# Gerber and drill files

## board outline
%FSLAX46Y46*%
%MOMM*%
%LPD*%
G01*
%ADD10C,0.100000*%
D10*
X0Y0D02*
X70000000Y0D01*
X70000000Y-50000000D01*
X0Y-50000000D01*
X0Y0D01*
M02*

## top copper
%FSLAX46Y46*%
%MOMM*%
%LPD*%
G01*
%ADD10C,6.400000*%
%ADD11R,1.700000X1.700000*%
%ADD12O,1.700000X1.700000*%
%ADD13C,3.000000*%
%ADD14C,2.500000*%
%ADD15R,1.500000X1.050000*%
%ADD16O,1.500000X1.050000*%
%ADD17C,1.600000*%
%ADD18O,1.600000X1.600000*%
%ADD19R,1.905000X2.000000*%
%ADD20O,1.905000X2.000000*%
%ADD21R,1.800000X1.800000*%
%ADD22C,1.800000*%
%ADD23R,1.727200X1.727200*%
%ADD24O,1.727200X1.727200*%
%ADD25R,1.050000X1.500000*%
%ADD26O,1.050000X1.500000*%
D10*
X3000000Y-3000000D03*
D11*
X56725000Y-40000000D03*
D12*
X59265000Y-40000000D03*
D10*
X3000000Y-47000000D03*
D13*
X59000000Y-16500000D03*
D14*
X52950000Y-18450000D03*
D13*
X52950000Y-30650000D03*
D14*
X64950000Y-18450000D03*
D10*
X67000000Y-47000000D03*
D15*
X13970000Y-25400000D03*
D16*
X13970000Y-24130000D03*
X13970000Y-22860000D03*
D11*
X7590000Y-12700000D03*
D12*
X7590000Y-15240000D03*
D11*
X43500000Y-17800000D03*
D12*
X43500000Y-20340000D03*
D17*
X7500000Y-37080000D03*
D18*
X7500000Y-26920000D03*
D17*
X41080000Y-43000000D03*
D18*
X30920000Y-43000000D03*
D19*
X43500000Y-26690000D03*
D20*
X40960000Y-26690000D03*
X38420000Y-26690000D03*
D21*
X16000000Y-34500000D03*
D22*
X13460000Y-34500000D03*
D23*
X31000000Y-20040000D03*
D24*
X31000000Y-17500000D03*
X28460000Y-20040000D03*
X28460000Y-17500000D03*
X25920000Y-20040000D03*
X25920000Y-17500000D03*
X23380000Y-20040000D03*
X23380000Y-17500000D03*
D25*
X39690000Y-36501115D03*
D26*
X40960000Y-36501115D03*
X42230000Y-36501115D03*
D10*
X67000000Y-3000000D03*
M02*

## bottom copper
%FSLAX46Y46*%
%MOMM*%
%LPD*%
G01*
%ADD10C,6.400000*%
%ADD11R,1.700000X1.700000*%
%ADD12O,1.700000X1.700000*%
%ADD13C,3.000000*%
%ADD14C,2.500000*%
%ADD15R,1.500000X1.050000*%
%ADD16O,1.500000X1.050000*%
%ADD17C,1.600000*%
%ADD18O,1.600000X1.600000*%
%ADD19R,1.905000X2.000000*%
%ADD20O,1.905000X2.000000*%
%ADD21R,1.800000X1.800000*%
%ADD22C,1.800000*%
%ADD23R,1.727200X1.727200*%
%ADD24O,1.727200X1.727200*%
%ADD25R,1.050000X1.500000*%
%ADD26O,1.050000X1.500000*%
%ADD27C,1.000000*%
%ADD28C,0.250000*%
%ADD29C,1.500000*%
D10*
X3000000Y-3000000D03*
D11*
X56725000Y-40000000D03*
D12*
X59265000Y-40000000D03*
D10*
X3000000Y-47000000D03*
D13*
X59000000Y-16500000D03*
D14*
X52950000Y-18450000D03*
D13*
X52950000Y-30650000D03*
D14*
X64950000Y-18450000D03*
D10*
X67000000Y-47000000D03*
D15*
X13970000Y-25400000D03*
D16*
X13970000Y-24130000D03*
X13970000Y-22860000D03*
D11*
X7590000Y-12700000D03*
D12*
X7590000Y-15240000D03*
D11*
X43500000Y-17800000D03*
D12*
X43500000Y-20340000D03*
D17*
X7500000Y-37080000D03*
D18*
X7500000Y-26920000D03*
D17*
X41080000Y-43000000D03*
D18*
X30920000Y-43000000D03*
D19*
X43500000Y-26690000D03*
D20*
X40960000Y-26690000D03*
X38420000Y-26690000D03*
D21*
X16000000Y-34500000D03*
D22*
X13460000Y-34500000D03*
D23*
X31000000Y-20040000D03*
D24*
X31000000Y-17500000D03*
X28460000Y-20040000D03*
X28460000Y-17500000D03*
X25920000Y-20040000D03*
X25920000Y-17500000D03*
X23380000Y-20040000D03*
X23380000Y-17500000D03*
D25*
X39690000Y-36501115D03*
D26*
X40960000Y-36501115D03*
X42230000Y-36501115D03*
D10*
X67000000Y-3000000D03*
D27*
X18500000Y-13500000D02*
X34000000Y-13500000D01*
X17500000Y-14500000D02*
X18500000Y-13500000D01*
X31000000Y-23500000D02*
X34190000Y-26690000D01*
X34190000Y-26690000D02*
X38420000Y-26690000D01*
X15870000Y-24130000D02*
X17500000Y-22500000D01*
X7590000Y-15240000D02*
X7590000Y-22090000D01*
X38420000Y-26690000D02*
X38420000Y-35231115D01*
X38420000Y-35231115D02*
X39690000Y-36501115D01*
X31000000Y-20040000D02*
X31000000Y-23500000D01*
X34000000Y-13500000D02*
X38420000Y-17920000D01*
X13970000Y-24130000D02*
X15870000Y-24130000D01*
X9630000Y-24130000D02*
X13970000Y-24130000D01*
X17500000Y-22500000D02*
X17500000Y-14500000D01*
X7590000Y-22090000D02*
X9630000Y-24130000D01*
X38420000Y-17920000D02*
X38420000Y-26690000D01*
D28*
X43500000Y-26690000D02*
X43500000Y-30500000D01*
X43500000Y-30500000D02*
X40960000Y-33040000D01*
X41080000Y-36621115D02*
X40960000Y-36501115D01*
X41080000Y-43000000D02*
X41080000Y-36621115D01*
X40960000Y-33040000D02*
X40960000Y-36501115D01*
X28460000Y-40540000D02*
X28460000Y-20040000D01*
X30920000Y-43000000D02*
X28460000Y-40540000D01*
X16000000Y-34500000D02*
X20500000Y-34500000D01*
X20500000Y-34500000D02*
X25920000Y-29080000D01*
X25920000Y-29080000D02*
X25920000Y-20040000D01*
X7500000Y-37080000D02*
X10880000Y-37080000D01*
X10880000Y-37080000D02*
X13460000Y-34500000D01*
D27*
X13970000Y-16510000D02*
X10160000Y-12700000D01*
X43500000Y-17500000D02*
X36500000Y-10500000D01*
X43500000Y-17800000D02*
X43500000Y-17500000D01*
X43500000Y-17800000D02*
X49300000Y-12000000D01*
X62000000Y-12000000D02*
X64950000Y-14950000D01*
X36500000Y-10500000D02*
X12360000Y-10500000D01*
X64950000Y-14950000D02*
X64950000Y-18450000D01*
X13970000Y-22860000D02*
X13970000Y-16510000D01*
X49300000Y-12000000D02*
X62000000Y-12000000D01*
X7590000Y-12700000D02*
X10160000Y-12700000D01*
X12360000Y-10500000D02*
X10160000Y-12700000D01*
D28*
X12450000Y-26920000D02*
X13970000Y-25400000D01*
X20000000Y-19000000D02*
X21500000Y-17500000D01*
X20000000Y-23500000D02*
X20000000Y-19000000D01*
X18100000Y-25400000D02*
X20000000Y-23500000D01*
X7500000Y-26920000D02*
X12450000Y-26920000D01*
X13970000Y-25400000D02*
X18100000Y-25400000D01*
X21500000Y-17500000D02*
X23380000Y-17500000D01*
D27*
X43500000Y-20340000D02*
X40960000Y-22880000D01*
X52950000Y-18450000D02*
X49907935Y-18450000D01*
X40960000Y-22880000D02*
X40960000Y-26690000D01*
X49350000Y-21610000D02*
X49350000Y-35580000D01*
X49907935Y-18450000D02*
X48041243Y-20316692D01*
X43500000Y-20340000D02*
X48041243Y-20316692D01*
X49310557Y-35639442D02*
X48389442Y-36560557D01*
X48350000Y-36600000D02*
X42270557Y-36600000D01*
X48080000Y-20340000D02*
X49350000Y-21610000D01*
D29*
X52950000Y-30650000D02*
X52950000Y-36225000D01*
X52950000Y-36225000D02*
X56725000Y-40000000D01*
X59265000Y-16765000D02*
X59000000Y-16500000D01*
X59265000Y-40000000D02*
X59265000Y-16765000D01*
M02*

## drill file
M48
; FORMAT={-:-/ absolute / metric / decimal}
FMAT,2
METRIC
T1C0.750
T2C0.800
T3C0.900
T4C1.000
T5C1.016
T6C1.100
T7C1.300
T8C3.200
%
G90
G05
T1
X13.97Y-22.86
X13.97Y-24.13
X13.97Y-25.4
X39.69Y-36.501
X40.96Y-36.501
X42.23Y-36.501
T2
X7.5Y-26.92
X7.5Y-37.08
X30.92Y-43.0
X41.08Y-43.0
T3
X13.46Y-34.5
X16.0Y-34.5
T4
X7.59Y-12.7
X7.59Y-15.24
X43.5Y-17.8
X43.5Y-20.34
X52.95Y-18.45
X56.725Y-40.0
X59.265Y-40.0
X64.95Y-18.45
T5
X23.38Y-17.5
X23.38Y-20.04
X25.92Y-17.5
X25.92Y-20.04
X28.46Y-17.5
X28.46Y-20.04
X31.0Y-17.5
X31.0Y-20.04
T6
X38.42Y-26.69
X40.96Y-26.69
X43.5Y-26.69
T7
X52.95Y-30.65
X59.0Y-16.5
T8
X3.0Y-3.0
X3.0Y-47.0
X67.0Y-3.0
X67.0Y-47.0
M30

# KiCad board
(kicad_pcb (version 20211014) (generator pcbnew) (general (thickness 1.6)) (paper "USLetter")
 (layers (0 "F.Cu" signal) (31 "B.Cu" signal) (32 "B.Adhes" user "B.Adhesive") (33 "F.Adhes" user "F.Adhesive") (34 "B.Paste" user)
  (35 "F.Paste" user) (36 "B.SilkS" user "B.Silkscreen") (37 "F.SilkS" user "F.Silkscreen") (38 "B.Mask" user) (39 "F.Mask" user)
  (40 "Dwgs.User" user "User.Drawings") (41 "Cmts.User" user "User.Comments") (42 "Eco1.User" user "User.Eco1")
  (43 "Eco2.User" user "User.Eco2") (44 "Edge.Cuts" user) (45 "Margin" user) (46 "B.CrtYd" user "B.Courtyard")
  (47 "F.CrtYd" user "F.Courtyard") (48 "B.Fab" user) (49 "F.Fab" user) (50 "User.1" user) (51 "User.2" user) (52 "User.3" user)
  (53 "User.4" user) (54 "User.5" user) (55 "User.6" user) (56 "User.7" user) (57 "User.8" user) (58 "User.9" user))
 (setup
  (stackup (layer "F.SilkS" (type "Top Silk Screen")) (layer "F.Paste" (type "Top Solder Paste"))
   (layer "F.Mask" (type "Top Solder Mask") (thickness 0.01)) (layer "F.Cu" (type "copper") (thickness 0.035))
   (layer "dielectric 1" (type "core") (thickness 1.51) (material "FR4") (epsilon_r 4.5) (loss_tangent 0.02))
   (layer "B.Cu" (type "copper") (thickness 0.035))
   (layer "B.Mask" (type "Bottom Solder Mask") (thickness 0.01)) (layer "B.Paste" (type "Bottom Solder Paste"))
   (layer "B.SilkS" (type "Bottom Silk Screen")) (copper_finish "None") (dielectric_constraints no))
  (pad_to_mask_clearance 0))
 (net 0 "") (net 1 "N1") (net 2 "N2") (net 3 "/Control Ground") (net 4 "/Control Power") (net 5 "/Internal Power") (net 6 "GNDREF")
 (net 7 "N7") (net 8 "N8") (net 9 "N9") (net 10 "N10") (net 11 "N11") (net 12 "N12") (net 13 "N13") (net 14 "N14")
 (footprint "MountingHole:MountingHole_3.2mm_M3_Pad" (layer "F.Cu") (at 3 3)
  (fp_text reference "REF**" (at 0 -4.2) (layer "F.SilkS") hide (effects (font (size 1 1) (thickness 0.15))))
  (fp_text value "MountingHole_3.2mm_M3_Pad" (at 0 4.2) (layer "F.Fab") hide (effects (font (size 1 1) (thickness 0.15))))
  (pad "1" thru_hole circle (at 0 0) (size 6.4 6.4) (drill 3.2) (layers *.Cu *.Mask)))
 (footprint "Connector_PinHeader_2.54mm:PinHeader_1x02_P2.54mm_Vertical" (layer "F.Cu") (at 56.725 40 90)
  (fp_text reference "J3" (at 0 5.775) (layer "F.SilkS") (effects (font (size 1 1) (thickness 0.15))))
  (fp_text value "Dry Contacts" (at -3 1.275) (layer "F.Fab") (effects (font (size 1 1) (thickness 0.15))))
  (pad "1" thru_hole rect (at 0 0 90) (size 1.7 1.7) (drill 1) (layers *.Cu *.Mask) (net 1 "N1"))
  (pad "2" thru_hole oval (at 0 2.54 90) (size 1.7 1.7) (drill 1) (layers *.Cu *.Mask) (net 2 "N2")))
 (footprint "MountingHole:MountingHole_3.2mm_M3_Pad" (layer "F.Cu") (at 3 47)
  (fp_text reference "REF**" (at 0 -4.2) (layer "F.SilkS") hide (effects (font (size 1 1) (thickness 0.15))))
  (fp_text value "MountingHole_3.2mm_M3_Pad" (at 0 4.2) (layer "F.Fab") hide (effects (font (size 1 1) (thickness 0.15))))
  (pad "1" thru_hole circle (at 0 0) (size 6.4 6.4) (drill 3.2) (layers *.Cu *.Mask)))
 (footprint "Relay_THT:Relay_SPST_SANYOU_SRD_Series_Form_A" (layer "F.Cu") (at 59 16.5 -90)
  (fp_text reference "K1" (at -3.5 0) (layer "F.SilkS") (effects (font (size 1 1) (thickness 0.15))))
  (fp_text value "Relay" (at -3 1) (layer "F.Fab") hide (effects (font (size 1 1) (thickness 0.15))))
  (pad "1" thru_hole circle (at 0 0) (size 3 3) (drill 1.3) (layers *.Cu *.Mask) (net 2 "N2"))
  (pad "2" thru_hole circle (at 1.95 6.05) (size 2.5 2.5) (drill 1) (layers *.Cu *.Mask) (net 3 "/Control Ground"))
  (pad "3" thru_hole circle (at 14.15 6.05) (size 3 3) (drill 1.3) (layers *.Cu *.Mask) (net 1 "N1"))
  (pad "5" thru_hole circle (at 1.95 -5.95) (size 2.5 2.5) (drill 1) (layers *.Cu *.Mask) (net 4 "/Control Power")))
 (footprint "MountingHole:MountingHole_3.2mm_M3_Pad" (layer "F.Cu") (at 67 47)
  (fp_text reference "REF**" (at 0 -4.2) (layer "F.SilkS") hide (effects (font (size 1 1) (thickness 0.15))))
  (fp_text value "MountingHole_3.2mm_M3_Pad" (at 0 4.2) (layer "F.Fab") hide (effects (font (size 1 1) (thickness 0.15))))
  (pad "1" thru_hole circle (at 0 0) (size 6.4 6.4) (drill 3.2) (layers *.Cu *.Mask)))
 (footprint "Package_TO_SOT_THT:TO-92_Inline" (layer "F.Cu") (at 13.97 25.4 90)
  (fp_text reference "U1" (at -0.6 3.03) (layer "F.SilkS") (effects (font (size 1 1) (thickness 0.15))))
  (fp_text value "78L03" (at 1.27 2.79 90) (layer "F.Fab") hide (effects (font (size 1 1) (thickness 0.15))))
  (pad "1" thru_hole rect (at 0 0 90) (size 1.05 1.5) (drill 0.75) (layers *.Cu *.Mask) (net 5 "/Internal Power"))
  (pad "2" thru_hole oval (at 1.27 0 90) (size 1.05 1.5) (drill 0.75) (layers *.Cu *.Mask) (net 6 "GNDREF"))
  (pad "3" thru_hole oval (at 2.54 0 90) (size 1.05 1.5) (drill 0.75) (layers *.Cu *.Mask) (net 4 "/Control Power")))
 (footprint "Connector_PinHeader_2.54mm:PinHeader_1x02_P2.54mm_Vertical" (layer "F.Cu") (at 7.59 12.7)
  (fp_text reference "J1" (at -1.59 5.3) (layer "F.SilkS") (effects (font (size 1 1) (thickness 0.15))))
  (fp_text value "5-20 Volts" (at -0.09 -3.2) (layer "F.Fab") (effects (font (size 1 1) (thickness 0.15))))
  (pad "1" thru_hole rect (at 0 0) (size 1.7 1.7) (drill 1) (layers *.Cu *.Mask) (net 4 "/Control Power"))
  (pad "2" thru_hole oval (at 0 2.54) (size 1.7 1.7) (drill 1) (layers *.Cu *.Mask) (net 6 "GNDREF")))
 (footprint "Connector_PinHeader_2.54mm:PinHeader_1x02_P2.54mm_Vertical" (layer "F.Cu") (at 43.5 17.8)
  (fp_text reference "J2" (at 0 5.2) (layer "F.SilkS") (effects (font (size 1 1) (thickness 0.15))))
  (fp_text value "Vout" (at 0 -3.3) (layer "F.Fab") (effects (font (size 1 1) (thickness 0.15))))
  (pad "1" thru_hole rect (at 0 0) (size 1.7 1.7) (drill 1) (layers *.Cu *.Mask) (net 4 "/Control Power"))
  (pad "2" thru_hole oval (at 0 2.54) (size 1.7 1.7) (drill 1) (layers *.Cu *.Mask) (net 3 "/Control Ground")))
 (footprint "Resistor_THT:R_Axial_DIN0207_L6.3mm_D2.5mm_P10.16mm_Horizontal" (layer "F.Cu") (at 7.5 37.08 90)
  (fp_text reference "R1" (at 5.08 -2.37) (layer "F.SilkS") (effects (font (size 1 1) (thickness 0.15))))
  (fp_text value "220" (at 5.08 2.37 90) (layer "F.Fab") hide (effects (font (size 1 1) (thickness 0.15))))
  (pad "1" thru_hole circle (at 0 0 90) (size 1.6 1.6) (drill 0.8) (layers *.Cu *.Mask) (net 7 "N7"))
  (pad "2" thru_hole oval (at 10.16 0 90) (size 1.6 1.6) (drill 0.8) (layers *.Cu *.Mask) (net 5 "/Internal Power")))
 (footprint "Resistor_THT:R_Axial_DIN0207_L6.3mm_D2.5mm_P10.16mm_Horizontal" (layer "F.Cu") (at 41.08 43 180)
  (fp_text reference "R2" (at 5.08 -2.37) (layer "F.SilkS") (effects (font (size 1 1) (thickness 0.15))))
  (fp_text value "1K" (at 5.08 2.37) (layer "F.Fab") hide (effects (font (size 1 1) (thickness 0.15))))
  (pad "1" thru_hole circle (at 0 0 180) (size 1.6 1.6) (drill 0.8) (layers *.Cu *.Mask) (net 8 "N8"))
  (pad "2" thru_hole oval (at 10.16 0 180) (size 1.6 1.6) (drill 0.8) (layers *.Cu *.Mask) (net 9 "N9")))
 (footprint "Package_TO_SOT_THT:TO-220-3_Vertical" (layer "F.Cu") (at 43.5 26.69 180)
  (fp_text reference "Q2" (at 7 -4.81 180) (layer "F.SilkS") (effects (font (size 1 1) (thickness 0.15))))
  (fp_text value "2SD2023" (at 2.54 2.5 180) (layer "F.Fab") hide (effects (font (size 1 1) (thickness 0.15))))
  (pad "1" thru_hole rect (at 0 0 180) (size 1.905 2) (drill 1.1) (layers *.Cu *.Mask) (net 8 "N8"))
  (pad "2" thru_hole oval (at 2.54 0 180) (size 1.905 2) (drill 1.1) (layers *.Cu *.Mask) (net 3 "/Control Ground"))
  (pad "3" thru_hole oval (at 5.08 0 180) (size 1.905 2) (drill 1.1) (layers *.Cu *.Mask) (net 6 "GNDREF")))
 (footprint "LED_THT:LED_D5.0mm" (layer "F.Cu") (at 16 34.5 180)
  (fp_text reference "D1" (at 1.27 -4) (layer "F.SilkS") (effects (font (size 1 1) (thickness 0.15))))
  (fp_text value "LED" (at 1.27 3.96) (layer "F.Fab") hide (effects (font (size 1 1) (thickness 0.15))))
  (pad "1" thru_hole rect (at 0 0 180) (size 1.8 1.8) (drill 0.9) (layers *.Cu *.Mask) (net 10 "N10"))
  (pad "2" thru_hole circle (at 2.54 0 180) (size 1.8 1.8) (drill 0.9) (layers *.Cu *.Mask) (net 7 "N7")))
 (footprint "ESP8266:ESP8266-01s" (layer "F.Cu") (at 31 17.5 -90)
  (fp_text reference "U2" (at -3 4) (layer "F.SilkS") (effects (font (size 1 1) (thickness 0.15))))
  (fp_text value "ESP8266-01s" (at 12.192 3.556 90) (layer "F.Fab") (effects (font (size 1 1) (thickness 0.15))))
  (pad "1" thru_hole rect (at 2.54 0 270) (size 1.7272 1.7272) (drill 1.016) (layers *.Cu *.Mask) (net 6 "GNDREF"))
  (pad "2" thru_hole oval (at 0 0 270) (size 1.7272 1.7272) (drill 1.016) (layers *.Cu *.Mask) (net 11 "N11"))
  (pad "3" thru_hole oval (at 2.54 2.54 270) (size 1.7272 1.7272) (drill 1.016) (layers *.Cu *.Mask) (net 9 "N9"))
  (pad "4" thru_hole oval (at 0 2.54 270) (size 1.7272 1.7272) (drill 1.016) (layers *.Cu *.Mask) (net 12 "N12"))
  (pad "5" thru_hole oval (at 2.54 5.08 270) (size 1.7272 1.7272) (drill 1.016) (layers *.Cu *.Mask) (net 10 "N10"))
  (pad "6" thru_hole oval (at 0 5.08 270) (size 1.7272 1.7272) (drill 1.016) (layers *.Cu *.Mask) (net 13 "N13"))
  (pad "7" thru_hole oval (at 2.54 7.62 270) (size 1.7272 1.7272) (drill 1.016) (layers *.Cu *.Mask) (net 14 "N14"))
  (pad "8" thru_hole oval (at 0 7.62 270) (size 1.7272 1.7272) (drill 1.016) (layers *.Cu *.Mask) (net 5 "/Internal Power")))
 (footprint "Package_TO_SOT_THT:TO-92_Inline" (layer "F.Cu") (at 39.69 36.501115)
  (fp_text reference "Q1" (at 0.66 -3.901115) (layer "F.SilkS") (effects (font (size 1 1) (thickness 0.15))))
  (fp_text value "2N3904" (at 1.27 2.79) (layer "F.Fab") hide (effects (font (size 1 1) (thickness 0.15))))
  (pad "1" thru_hole rect (at 0 0) (size 1.05 1.5) (drill 0.75) (layers *.Cu *.Mask) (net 6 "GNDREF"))
  (pad "2" thru_hole oval (at 1.27 0) (size 1.05 1.5) (drill 0.75) (layers *.Cu *.Mask) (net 8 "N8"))
  (pad "3" thru_hole oval (at 2.54 0) (size 1.05 1.5) (drill 0.75) (layers *.Cu *.Mask) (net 3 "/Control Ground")))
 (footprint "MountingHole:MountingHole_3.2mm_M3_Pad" (layer "F.Cu") (at 67 3)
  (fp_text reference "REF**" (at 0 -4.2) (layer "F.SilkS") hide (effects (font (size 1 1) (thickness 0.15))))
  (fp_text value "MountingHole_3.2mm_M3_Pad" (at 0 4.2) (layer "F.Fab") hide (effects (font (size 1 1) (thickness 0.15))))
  (pad "1" thru_hole circle (at 0 0) (size 6.4 6.4) (drill 3.2) (layers *.Cu *.Mask)))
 (gr_rect (start 0 0) (end 70 50) (layer "Edge.Cuts") (width 0.1) (fill none))
 (segment (start 18.5 13.5) (end 34 13.5) (width 1) (layer "B.Cu") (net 6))
 (segment (start 17.5 14.5) (end 18.5 13.5) (width 1) (layer "B.Cu") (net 6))
 (segment (start 31 23.5) (end 34.19 26.69) (width 1) (layer "B.Cu") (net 6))
 (segment (start 34.19 26.69) (end 38.42 26.69) (width 1) (layer "B.Cu") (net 6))
 (segment (start 15.87 24.13) (end 17.5 22.5) (width 1) (layer "B.Cu") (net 6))
 (segment (start 7.59 15.24) (end 7.59 22.09) (width 1) (layer "B.Cu") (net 6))
 (segment (start 38.42 26.69) (end 38.42 35.231115) (width 1) (layer "B.Cu") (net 6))
 (segment (start 38.42 35.231115) (end 39.69 36.501115) (width 1) (layer "B.Cu") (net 6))
 (segment (start 31 20.04) (end 31 23.5) (width 1) (layer "B.Cu") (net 6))
 (segment (start 34 13.5) (end 38.42 17.92) (width 1) (layer "B.Cu") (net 6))
 (segment (start 13.97 24.13) (end 15.87 24.13) (width 1) (layer "B.Cu") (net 6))
 (segment (start 9.63 24.13) (end 13.97 24.13) (width 1) (layer "B.Cu") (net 6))
 (segment (start 17.5 22.5) (end 17.5 14.5) (width 1) (layer "B.Cu") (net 6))
 (segment (start 7.59 22.09) (end 9.63 24.13) (width 1) (layer "B.Cu") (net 6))
 (segment (start 38.42 17.92) (end 38.42 26.69) (width 1) (layer "B.Cu") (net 6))
 (segment (start 43.5 26.69) (end 43.5 30.5) (width 0.25) (layer "B.Cu") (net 8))
 (segment (start 43.5 30.5) (end 40.96 33.04) (width 0.25) (layer "B.Cu") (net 8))
 (segment (start 41.08 36.621115) (end 40.96 36.501115) (width 0.25) (layer "B.Cu") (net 8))
 (segment (start 41.08 43) (end 41.08 36.621115) (width 0.25) (layer "B.Cu") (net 8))
 (segment (start 40.96 33.04) (end 40.96 36.501115) (width 0.25) (layer "B.Cu") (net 8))
 (segment (start 28.46 40.54) (end 28.46 20.04) (width 0.25) (layer "B.Cu") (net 9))
 (segment (start 30.92 43) (end 28.46 40.54) (width 0.25) (layer "B.Cu") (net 9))
 (segment (start 16 34.5) (end 20.5 34.5) (width 0.25) (layer "B.Cu") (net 10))
 (segment (start 20.5 34.5) (end 25.92 29.08) (width 0.25) (layer "B.Cu") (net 10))
 (segment (start 25.92 29.08) (end 25.92 20.04) (width 0.25) (layer "B.Cu") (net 10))
 (segment (start 7.5 37.08) (end 10.88 37.08) (width 0.25) (layer "B.Cu") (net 7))
 (segment (start 10.88 37.08) (end 13.46 34.5) (width 0.25) (layer "B.Cu") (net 7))
 (segment (start 13.97 16.51) (end 10.16 12.7) (width 1) (layer "B.Cu") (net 4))
 (segment (start 43.5 17.5) (end 36.5 10.5) (width 1) (layer "B.Cu") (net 4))
 (segment (start 43.5 17.8) (end 43.5 17.5) (width 1) (layer "B.Cu") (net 4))
 (segment (start 43.5 17.8) (end 49.3 12) (width 1) (layer "B.Cu") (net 4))
 (segment (start 62 12) (end 64.95 14.95) (width 1) (layer "B.Cu") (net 4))
 (segment (start 36.5 10.5) (end 12.36 10.5) (width 1) (layer "B.Cu") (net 4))
 (segment (start 64.95 14.95) (end 64.95 18.45) (width 1) (layer "B.Cu") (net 4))
 (segment (start 13.97 22.86) (end 13.97 16.51) (width 1) (layer "B.Cu") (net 4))
 (segment (start 49.3 12) (end 62 12) (width 1) (layer "B.Cu") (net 4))
 (segment (start 7.59 12.7) (end 10.16 12.7) (width 1) (layer "B.Cu") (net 4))
 (segment (start 12.36 10.5) (end 10.16 12.7) (width 1) (layer "B.Cu") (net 4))
 (segment (start 12.45 26.92) (end 13.97 25.4) (width 0.25) (layer "B.Cu") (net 5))
 (segment (start 20 19) (end 21.5 17.5) (width 0.25) (layer "B.Cu") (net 5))
 (segment (start 20 23.5) (end 20 19) (width 0.25) (layer "B.Cu") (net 5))
 (segment (start 18.1 25.4) (end 20 23.5) (width 0.25) (layer "B.Cu") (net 5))
 (segment (start 7.5 26.92) (end 12.45 26.92) (width 0.25) (layer "B.Cu") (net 5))
 (segment (start 13.97 25.4) (end 18.1 25.4) (width 0.25) (layer "B.Cu") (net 5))
 (segment (start 21.5 17.5) (end 23.38 17.5) (width 0.25) (layer "B.Cu") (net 5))
 (segment (start 43.5 20.34) (end 40.96 22.88) (width 1) (layer "B.Cu") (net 3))
 (segment (start 52.95 18.45) (end 49.907935 18.45) (width 1) (layer "B.Cu") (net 3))
 (segment (start 40.96 22.88) (end 40.96 26.69) (width 1) (layer "B.Cu") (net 3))
 (segment (start 49.35 21.61) (end 49.35 35.58) (width 1) (layer "B.Cu") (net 3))
 (segment (start 49.907935 18.45) (end 48.041243 20.316692) (width 1) (layer "B.Cu") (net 3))
 (segment (start 43.5 20.34) (end 48.041243 20.316692) (width 1) (layer "B.Cu") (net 3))
 (segment (start 49.310557 35.639442) (end 48.389442 36.560557) (width 1) (layer "B.Cu") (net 3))
 (segment (start 48.35 36.6) (end 42.270557 36.6) (width 1) (layer "B.Cu") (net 3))
 (segment (start 48.08 20.34) (end 49.35 21.61) (width 1) (layer "B.Cu") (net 3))
 (segment (start 52.95 30.65) (end 52.95 36.225) (width 1.5) (layer "B.Cu") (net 1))
 (segment (start 52.95 36.225) (end 56.725 40) (width 1.5) (layer "B.Cu") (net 1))
 (segment (start 59.265 16.765) (end 59 16.5) (width 1.5) (layer "B.Cu") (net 2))
 (segment (start 59.265 40) (end 59.265 16.765) (width 1.5) (layer "B.Cu") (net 2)))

